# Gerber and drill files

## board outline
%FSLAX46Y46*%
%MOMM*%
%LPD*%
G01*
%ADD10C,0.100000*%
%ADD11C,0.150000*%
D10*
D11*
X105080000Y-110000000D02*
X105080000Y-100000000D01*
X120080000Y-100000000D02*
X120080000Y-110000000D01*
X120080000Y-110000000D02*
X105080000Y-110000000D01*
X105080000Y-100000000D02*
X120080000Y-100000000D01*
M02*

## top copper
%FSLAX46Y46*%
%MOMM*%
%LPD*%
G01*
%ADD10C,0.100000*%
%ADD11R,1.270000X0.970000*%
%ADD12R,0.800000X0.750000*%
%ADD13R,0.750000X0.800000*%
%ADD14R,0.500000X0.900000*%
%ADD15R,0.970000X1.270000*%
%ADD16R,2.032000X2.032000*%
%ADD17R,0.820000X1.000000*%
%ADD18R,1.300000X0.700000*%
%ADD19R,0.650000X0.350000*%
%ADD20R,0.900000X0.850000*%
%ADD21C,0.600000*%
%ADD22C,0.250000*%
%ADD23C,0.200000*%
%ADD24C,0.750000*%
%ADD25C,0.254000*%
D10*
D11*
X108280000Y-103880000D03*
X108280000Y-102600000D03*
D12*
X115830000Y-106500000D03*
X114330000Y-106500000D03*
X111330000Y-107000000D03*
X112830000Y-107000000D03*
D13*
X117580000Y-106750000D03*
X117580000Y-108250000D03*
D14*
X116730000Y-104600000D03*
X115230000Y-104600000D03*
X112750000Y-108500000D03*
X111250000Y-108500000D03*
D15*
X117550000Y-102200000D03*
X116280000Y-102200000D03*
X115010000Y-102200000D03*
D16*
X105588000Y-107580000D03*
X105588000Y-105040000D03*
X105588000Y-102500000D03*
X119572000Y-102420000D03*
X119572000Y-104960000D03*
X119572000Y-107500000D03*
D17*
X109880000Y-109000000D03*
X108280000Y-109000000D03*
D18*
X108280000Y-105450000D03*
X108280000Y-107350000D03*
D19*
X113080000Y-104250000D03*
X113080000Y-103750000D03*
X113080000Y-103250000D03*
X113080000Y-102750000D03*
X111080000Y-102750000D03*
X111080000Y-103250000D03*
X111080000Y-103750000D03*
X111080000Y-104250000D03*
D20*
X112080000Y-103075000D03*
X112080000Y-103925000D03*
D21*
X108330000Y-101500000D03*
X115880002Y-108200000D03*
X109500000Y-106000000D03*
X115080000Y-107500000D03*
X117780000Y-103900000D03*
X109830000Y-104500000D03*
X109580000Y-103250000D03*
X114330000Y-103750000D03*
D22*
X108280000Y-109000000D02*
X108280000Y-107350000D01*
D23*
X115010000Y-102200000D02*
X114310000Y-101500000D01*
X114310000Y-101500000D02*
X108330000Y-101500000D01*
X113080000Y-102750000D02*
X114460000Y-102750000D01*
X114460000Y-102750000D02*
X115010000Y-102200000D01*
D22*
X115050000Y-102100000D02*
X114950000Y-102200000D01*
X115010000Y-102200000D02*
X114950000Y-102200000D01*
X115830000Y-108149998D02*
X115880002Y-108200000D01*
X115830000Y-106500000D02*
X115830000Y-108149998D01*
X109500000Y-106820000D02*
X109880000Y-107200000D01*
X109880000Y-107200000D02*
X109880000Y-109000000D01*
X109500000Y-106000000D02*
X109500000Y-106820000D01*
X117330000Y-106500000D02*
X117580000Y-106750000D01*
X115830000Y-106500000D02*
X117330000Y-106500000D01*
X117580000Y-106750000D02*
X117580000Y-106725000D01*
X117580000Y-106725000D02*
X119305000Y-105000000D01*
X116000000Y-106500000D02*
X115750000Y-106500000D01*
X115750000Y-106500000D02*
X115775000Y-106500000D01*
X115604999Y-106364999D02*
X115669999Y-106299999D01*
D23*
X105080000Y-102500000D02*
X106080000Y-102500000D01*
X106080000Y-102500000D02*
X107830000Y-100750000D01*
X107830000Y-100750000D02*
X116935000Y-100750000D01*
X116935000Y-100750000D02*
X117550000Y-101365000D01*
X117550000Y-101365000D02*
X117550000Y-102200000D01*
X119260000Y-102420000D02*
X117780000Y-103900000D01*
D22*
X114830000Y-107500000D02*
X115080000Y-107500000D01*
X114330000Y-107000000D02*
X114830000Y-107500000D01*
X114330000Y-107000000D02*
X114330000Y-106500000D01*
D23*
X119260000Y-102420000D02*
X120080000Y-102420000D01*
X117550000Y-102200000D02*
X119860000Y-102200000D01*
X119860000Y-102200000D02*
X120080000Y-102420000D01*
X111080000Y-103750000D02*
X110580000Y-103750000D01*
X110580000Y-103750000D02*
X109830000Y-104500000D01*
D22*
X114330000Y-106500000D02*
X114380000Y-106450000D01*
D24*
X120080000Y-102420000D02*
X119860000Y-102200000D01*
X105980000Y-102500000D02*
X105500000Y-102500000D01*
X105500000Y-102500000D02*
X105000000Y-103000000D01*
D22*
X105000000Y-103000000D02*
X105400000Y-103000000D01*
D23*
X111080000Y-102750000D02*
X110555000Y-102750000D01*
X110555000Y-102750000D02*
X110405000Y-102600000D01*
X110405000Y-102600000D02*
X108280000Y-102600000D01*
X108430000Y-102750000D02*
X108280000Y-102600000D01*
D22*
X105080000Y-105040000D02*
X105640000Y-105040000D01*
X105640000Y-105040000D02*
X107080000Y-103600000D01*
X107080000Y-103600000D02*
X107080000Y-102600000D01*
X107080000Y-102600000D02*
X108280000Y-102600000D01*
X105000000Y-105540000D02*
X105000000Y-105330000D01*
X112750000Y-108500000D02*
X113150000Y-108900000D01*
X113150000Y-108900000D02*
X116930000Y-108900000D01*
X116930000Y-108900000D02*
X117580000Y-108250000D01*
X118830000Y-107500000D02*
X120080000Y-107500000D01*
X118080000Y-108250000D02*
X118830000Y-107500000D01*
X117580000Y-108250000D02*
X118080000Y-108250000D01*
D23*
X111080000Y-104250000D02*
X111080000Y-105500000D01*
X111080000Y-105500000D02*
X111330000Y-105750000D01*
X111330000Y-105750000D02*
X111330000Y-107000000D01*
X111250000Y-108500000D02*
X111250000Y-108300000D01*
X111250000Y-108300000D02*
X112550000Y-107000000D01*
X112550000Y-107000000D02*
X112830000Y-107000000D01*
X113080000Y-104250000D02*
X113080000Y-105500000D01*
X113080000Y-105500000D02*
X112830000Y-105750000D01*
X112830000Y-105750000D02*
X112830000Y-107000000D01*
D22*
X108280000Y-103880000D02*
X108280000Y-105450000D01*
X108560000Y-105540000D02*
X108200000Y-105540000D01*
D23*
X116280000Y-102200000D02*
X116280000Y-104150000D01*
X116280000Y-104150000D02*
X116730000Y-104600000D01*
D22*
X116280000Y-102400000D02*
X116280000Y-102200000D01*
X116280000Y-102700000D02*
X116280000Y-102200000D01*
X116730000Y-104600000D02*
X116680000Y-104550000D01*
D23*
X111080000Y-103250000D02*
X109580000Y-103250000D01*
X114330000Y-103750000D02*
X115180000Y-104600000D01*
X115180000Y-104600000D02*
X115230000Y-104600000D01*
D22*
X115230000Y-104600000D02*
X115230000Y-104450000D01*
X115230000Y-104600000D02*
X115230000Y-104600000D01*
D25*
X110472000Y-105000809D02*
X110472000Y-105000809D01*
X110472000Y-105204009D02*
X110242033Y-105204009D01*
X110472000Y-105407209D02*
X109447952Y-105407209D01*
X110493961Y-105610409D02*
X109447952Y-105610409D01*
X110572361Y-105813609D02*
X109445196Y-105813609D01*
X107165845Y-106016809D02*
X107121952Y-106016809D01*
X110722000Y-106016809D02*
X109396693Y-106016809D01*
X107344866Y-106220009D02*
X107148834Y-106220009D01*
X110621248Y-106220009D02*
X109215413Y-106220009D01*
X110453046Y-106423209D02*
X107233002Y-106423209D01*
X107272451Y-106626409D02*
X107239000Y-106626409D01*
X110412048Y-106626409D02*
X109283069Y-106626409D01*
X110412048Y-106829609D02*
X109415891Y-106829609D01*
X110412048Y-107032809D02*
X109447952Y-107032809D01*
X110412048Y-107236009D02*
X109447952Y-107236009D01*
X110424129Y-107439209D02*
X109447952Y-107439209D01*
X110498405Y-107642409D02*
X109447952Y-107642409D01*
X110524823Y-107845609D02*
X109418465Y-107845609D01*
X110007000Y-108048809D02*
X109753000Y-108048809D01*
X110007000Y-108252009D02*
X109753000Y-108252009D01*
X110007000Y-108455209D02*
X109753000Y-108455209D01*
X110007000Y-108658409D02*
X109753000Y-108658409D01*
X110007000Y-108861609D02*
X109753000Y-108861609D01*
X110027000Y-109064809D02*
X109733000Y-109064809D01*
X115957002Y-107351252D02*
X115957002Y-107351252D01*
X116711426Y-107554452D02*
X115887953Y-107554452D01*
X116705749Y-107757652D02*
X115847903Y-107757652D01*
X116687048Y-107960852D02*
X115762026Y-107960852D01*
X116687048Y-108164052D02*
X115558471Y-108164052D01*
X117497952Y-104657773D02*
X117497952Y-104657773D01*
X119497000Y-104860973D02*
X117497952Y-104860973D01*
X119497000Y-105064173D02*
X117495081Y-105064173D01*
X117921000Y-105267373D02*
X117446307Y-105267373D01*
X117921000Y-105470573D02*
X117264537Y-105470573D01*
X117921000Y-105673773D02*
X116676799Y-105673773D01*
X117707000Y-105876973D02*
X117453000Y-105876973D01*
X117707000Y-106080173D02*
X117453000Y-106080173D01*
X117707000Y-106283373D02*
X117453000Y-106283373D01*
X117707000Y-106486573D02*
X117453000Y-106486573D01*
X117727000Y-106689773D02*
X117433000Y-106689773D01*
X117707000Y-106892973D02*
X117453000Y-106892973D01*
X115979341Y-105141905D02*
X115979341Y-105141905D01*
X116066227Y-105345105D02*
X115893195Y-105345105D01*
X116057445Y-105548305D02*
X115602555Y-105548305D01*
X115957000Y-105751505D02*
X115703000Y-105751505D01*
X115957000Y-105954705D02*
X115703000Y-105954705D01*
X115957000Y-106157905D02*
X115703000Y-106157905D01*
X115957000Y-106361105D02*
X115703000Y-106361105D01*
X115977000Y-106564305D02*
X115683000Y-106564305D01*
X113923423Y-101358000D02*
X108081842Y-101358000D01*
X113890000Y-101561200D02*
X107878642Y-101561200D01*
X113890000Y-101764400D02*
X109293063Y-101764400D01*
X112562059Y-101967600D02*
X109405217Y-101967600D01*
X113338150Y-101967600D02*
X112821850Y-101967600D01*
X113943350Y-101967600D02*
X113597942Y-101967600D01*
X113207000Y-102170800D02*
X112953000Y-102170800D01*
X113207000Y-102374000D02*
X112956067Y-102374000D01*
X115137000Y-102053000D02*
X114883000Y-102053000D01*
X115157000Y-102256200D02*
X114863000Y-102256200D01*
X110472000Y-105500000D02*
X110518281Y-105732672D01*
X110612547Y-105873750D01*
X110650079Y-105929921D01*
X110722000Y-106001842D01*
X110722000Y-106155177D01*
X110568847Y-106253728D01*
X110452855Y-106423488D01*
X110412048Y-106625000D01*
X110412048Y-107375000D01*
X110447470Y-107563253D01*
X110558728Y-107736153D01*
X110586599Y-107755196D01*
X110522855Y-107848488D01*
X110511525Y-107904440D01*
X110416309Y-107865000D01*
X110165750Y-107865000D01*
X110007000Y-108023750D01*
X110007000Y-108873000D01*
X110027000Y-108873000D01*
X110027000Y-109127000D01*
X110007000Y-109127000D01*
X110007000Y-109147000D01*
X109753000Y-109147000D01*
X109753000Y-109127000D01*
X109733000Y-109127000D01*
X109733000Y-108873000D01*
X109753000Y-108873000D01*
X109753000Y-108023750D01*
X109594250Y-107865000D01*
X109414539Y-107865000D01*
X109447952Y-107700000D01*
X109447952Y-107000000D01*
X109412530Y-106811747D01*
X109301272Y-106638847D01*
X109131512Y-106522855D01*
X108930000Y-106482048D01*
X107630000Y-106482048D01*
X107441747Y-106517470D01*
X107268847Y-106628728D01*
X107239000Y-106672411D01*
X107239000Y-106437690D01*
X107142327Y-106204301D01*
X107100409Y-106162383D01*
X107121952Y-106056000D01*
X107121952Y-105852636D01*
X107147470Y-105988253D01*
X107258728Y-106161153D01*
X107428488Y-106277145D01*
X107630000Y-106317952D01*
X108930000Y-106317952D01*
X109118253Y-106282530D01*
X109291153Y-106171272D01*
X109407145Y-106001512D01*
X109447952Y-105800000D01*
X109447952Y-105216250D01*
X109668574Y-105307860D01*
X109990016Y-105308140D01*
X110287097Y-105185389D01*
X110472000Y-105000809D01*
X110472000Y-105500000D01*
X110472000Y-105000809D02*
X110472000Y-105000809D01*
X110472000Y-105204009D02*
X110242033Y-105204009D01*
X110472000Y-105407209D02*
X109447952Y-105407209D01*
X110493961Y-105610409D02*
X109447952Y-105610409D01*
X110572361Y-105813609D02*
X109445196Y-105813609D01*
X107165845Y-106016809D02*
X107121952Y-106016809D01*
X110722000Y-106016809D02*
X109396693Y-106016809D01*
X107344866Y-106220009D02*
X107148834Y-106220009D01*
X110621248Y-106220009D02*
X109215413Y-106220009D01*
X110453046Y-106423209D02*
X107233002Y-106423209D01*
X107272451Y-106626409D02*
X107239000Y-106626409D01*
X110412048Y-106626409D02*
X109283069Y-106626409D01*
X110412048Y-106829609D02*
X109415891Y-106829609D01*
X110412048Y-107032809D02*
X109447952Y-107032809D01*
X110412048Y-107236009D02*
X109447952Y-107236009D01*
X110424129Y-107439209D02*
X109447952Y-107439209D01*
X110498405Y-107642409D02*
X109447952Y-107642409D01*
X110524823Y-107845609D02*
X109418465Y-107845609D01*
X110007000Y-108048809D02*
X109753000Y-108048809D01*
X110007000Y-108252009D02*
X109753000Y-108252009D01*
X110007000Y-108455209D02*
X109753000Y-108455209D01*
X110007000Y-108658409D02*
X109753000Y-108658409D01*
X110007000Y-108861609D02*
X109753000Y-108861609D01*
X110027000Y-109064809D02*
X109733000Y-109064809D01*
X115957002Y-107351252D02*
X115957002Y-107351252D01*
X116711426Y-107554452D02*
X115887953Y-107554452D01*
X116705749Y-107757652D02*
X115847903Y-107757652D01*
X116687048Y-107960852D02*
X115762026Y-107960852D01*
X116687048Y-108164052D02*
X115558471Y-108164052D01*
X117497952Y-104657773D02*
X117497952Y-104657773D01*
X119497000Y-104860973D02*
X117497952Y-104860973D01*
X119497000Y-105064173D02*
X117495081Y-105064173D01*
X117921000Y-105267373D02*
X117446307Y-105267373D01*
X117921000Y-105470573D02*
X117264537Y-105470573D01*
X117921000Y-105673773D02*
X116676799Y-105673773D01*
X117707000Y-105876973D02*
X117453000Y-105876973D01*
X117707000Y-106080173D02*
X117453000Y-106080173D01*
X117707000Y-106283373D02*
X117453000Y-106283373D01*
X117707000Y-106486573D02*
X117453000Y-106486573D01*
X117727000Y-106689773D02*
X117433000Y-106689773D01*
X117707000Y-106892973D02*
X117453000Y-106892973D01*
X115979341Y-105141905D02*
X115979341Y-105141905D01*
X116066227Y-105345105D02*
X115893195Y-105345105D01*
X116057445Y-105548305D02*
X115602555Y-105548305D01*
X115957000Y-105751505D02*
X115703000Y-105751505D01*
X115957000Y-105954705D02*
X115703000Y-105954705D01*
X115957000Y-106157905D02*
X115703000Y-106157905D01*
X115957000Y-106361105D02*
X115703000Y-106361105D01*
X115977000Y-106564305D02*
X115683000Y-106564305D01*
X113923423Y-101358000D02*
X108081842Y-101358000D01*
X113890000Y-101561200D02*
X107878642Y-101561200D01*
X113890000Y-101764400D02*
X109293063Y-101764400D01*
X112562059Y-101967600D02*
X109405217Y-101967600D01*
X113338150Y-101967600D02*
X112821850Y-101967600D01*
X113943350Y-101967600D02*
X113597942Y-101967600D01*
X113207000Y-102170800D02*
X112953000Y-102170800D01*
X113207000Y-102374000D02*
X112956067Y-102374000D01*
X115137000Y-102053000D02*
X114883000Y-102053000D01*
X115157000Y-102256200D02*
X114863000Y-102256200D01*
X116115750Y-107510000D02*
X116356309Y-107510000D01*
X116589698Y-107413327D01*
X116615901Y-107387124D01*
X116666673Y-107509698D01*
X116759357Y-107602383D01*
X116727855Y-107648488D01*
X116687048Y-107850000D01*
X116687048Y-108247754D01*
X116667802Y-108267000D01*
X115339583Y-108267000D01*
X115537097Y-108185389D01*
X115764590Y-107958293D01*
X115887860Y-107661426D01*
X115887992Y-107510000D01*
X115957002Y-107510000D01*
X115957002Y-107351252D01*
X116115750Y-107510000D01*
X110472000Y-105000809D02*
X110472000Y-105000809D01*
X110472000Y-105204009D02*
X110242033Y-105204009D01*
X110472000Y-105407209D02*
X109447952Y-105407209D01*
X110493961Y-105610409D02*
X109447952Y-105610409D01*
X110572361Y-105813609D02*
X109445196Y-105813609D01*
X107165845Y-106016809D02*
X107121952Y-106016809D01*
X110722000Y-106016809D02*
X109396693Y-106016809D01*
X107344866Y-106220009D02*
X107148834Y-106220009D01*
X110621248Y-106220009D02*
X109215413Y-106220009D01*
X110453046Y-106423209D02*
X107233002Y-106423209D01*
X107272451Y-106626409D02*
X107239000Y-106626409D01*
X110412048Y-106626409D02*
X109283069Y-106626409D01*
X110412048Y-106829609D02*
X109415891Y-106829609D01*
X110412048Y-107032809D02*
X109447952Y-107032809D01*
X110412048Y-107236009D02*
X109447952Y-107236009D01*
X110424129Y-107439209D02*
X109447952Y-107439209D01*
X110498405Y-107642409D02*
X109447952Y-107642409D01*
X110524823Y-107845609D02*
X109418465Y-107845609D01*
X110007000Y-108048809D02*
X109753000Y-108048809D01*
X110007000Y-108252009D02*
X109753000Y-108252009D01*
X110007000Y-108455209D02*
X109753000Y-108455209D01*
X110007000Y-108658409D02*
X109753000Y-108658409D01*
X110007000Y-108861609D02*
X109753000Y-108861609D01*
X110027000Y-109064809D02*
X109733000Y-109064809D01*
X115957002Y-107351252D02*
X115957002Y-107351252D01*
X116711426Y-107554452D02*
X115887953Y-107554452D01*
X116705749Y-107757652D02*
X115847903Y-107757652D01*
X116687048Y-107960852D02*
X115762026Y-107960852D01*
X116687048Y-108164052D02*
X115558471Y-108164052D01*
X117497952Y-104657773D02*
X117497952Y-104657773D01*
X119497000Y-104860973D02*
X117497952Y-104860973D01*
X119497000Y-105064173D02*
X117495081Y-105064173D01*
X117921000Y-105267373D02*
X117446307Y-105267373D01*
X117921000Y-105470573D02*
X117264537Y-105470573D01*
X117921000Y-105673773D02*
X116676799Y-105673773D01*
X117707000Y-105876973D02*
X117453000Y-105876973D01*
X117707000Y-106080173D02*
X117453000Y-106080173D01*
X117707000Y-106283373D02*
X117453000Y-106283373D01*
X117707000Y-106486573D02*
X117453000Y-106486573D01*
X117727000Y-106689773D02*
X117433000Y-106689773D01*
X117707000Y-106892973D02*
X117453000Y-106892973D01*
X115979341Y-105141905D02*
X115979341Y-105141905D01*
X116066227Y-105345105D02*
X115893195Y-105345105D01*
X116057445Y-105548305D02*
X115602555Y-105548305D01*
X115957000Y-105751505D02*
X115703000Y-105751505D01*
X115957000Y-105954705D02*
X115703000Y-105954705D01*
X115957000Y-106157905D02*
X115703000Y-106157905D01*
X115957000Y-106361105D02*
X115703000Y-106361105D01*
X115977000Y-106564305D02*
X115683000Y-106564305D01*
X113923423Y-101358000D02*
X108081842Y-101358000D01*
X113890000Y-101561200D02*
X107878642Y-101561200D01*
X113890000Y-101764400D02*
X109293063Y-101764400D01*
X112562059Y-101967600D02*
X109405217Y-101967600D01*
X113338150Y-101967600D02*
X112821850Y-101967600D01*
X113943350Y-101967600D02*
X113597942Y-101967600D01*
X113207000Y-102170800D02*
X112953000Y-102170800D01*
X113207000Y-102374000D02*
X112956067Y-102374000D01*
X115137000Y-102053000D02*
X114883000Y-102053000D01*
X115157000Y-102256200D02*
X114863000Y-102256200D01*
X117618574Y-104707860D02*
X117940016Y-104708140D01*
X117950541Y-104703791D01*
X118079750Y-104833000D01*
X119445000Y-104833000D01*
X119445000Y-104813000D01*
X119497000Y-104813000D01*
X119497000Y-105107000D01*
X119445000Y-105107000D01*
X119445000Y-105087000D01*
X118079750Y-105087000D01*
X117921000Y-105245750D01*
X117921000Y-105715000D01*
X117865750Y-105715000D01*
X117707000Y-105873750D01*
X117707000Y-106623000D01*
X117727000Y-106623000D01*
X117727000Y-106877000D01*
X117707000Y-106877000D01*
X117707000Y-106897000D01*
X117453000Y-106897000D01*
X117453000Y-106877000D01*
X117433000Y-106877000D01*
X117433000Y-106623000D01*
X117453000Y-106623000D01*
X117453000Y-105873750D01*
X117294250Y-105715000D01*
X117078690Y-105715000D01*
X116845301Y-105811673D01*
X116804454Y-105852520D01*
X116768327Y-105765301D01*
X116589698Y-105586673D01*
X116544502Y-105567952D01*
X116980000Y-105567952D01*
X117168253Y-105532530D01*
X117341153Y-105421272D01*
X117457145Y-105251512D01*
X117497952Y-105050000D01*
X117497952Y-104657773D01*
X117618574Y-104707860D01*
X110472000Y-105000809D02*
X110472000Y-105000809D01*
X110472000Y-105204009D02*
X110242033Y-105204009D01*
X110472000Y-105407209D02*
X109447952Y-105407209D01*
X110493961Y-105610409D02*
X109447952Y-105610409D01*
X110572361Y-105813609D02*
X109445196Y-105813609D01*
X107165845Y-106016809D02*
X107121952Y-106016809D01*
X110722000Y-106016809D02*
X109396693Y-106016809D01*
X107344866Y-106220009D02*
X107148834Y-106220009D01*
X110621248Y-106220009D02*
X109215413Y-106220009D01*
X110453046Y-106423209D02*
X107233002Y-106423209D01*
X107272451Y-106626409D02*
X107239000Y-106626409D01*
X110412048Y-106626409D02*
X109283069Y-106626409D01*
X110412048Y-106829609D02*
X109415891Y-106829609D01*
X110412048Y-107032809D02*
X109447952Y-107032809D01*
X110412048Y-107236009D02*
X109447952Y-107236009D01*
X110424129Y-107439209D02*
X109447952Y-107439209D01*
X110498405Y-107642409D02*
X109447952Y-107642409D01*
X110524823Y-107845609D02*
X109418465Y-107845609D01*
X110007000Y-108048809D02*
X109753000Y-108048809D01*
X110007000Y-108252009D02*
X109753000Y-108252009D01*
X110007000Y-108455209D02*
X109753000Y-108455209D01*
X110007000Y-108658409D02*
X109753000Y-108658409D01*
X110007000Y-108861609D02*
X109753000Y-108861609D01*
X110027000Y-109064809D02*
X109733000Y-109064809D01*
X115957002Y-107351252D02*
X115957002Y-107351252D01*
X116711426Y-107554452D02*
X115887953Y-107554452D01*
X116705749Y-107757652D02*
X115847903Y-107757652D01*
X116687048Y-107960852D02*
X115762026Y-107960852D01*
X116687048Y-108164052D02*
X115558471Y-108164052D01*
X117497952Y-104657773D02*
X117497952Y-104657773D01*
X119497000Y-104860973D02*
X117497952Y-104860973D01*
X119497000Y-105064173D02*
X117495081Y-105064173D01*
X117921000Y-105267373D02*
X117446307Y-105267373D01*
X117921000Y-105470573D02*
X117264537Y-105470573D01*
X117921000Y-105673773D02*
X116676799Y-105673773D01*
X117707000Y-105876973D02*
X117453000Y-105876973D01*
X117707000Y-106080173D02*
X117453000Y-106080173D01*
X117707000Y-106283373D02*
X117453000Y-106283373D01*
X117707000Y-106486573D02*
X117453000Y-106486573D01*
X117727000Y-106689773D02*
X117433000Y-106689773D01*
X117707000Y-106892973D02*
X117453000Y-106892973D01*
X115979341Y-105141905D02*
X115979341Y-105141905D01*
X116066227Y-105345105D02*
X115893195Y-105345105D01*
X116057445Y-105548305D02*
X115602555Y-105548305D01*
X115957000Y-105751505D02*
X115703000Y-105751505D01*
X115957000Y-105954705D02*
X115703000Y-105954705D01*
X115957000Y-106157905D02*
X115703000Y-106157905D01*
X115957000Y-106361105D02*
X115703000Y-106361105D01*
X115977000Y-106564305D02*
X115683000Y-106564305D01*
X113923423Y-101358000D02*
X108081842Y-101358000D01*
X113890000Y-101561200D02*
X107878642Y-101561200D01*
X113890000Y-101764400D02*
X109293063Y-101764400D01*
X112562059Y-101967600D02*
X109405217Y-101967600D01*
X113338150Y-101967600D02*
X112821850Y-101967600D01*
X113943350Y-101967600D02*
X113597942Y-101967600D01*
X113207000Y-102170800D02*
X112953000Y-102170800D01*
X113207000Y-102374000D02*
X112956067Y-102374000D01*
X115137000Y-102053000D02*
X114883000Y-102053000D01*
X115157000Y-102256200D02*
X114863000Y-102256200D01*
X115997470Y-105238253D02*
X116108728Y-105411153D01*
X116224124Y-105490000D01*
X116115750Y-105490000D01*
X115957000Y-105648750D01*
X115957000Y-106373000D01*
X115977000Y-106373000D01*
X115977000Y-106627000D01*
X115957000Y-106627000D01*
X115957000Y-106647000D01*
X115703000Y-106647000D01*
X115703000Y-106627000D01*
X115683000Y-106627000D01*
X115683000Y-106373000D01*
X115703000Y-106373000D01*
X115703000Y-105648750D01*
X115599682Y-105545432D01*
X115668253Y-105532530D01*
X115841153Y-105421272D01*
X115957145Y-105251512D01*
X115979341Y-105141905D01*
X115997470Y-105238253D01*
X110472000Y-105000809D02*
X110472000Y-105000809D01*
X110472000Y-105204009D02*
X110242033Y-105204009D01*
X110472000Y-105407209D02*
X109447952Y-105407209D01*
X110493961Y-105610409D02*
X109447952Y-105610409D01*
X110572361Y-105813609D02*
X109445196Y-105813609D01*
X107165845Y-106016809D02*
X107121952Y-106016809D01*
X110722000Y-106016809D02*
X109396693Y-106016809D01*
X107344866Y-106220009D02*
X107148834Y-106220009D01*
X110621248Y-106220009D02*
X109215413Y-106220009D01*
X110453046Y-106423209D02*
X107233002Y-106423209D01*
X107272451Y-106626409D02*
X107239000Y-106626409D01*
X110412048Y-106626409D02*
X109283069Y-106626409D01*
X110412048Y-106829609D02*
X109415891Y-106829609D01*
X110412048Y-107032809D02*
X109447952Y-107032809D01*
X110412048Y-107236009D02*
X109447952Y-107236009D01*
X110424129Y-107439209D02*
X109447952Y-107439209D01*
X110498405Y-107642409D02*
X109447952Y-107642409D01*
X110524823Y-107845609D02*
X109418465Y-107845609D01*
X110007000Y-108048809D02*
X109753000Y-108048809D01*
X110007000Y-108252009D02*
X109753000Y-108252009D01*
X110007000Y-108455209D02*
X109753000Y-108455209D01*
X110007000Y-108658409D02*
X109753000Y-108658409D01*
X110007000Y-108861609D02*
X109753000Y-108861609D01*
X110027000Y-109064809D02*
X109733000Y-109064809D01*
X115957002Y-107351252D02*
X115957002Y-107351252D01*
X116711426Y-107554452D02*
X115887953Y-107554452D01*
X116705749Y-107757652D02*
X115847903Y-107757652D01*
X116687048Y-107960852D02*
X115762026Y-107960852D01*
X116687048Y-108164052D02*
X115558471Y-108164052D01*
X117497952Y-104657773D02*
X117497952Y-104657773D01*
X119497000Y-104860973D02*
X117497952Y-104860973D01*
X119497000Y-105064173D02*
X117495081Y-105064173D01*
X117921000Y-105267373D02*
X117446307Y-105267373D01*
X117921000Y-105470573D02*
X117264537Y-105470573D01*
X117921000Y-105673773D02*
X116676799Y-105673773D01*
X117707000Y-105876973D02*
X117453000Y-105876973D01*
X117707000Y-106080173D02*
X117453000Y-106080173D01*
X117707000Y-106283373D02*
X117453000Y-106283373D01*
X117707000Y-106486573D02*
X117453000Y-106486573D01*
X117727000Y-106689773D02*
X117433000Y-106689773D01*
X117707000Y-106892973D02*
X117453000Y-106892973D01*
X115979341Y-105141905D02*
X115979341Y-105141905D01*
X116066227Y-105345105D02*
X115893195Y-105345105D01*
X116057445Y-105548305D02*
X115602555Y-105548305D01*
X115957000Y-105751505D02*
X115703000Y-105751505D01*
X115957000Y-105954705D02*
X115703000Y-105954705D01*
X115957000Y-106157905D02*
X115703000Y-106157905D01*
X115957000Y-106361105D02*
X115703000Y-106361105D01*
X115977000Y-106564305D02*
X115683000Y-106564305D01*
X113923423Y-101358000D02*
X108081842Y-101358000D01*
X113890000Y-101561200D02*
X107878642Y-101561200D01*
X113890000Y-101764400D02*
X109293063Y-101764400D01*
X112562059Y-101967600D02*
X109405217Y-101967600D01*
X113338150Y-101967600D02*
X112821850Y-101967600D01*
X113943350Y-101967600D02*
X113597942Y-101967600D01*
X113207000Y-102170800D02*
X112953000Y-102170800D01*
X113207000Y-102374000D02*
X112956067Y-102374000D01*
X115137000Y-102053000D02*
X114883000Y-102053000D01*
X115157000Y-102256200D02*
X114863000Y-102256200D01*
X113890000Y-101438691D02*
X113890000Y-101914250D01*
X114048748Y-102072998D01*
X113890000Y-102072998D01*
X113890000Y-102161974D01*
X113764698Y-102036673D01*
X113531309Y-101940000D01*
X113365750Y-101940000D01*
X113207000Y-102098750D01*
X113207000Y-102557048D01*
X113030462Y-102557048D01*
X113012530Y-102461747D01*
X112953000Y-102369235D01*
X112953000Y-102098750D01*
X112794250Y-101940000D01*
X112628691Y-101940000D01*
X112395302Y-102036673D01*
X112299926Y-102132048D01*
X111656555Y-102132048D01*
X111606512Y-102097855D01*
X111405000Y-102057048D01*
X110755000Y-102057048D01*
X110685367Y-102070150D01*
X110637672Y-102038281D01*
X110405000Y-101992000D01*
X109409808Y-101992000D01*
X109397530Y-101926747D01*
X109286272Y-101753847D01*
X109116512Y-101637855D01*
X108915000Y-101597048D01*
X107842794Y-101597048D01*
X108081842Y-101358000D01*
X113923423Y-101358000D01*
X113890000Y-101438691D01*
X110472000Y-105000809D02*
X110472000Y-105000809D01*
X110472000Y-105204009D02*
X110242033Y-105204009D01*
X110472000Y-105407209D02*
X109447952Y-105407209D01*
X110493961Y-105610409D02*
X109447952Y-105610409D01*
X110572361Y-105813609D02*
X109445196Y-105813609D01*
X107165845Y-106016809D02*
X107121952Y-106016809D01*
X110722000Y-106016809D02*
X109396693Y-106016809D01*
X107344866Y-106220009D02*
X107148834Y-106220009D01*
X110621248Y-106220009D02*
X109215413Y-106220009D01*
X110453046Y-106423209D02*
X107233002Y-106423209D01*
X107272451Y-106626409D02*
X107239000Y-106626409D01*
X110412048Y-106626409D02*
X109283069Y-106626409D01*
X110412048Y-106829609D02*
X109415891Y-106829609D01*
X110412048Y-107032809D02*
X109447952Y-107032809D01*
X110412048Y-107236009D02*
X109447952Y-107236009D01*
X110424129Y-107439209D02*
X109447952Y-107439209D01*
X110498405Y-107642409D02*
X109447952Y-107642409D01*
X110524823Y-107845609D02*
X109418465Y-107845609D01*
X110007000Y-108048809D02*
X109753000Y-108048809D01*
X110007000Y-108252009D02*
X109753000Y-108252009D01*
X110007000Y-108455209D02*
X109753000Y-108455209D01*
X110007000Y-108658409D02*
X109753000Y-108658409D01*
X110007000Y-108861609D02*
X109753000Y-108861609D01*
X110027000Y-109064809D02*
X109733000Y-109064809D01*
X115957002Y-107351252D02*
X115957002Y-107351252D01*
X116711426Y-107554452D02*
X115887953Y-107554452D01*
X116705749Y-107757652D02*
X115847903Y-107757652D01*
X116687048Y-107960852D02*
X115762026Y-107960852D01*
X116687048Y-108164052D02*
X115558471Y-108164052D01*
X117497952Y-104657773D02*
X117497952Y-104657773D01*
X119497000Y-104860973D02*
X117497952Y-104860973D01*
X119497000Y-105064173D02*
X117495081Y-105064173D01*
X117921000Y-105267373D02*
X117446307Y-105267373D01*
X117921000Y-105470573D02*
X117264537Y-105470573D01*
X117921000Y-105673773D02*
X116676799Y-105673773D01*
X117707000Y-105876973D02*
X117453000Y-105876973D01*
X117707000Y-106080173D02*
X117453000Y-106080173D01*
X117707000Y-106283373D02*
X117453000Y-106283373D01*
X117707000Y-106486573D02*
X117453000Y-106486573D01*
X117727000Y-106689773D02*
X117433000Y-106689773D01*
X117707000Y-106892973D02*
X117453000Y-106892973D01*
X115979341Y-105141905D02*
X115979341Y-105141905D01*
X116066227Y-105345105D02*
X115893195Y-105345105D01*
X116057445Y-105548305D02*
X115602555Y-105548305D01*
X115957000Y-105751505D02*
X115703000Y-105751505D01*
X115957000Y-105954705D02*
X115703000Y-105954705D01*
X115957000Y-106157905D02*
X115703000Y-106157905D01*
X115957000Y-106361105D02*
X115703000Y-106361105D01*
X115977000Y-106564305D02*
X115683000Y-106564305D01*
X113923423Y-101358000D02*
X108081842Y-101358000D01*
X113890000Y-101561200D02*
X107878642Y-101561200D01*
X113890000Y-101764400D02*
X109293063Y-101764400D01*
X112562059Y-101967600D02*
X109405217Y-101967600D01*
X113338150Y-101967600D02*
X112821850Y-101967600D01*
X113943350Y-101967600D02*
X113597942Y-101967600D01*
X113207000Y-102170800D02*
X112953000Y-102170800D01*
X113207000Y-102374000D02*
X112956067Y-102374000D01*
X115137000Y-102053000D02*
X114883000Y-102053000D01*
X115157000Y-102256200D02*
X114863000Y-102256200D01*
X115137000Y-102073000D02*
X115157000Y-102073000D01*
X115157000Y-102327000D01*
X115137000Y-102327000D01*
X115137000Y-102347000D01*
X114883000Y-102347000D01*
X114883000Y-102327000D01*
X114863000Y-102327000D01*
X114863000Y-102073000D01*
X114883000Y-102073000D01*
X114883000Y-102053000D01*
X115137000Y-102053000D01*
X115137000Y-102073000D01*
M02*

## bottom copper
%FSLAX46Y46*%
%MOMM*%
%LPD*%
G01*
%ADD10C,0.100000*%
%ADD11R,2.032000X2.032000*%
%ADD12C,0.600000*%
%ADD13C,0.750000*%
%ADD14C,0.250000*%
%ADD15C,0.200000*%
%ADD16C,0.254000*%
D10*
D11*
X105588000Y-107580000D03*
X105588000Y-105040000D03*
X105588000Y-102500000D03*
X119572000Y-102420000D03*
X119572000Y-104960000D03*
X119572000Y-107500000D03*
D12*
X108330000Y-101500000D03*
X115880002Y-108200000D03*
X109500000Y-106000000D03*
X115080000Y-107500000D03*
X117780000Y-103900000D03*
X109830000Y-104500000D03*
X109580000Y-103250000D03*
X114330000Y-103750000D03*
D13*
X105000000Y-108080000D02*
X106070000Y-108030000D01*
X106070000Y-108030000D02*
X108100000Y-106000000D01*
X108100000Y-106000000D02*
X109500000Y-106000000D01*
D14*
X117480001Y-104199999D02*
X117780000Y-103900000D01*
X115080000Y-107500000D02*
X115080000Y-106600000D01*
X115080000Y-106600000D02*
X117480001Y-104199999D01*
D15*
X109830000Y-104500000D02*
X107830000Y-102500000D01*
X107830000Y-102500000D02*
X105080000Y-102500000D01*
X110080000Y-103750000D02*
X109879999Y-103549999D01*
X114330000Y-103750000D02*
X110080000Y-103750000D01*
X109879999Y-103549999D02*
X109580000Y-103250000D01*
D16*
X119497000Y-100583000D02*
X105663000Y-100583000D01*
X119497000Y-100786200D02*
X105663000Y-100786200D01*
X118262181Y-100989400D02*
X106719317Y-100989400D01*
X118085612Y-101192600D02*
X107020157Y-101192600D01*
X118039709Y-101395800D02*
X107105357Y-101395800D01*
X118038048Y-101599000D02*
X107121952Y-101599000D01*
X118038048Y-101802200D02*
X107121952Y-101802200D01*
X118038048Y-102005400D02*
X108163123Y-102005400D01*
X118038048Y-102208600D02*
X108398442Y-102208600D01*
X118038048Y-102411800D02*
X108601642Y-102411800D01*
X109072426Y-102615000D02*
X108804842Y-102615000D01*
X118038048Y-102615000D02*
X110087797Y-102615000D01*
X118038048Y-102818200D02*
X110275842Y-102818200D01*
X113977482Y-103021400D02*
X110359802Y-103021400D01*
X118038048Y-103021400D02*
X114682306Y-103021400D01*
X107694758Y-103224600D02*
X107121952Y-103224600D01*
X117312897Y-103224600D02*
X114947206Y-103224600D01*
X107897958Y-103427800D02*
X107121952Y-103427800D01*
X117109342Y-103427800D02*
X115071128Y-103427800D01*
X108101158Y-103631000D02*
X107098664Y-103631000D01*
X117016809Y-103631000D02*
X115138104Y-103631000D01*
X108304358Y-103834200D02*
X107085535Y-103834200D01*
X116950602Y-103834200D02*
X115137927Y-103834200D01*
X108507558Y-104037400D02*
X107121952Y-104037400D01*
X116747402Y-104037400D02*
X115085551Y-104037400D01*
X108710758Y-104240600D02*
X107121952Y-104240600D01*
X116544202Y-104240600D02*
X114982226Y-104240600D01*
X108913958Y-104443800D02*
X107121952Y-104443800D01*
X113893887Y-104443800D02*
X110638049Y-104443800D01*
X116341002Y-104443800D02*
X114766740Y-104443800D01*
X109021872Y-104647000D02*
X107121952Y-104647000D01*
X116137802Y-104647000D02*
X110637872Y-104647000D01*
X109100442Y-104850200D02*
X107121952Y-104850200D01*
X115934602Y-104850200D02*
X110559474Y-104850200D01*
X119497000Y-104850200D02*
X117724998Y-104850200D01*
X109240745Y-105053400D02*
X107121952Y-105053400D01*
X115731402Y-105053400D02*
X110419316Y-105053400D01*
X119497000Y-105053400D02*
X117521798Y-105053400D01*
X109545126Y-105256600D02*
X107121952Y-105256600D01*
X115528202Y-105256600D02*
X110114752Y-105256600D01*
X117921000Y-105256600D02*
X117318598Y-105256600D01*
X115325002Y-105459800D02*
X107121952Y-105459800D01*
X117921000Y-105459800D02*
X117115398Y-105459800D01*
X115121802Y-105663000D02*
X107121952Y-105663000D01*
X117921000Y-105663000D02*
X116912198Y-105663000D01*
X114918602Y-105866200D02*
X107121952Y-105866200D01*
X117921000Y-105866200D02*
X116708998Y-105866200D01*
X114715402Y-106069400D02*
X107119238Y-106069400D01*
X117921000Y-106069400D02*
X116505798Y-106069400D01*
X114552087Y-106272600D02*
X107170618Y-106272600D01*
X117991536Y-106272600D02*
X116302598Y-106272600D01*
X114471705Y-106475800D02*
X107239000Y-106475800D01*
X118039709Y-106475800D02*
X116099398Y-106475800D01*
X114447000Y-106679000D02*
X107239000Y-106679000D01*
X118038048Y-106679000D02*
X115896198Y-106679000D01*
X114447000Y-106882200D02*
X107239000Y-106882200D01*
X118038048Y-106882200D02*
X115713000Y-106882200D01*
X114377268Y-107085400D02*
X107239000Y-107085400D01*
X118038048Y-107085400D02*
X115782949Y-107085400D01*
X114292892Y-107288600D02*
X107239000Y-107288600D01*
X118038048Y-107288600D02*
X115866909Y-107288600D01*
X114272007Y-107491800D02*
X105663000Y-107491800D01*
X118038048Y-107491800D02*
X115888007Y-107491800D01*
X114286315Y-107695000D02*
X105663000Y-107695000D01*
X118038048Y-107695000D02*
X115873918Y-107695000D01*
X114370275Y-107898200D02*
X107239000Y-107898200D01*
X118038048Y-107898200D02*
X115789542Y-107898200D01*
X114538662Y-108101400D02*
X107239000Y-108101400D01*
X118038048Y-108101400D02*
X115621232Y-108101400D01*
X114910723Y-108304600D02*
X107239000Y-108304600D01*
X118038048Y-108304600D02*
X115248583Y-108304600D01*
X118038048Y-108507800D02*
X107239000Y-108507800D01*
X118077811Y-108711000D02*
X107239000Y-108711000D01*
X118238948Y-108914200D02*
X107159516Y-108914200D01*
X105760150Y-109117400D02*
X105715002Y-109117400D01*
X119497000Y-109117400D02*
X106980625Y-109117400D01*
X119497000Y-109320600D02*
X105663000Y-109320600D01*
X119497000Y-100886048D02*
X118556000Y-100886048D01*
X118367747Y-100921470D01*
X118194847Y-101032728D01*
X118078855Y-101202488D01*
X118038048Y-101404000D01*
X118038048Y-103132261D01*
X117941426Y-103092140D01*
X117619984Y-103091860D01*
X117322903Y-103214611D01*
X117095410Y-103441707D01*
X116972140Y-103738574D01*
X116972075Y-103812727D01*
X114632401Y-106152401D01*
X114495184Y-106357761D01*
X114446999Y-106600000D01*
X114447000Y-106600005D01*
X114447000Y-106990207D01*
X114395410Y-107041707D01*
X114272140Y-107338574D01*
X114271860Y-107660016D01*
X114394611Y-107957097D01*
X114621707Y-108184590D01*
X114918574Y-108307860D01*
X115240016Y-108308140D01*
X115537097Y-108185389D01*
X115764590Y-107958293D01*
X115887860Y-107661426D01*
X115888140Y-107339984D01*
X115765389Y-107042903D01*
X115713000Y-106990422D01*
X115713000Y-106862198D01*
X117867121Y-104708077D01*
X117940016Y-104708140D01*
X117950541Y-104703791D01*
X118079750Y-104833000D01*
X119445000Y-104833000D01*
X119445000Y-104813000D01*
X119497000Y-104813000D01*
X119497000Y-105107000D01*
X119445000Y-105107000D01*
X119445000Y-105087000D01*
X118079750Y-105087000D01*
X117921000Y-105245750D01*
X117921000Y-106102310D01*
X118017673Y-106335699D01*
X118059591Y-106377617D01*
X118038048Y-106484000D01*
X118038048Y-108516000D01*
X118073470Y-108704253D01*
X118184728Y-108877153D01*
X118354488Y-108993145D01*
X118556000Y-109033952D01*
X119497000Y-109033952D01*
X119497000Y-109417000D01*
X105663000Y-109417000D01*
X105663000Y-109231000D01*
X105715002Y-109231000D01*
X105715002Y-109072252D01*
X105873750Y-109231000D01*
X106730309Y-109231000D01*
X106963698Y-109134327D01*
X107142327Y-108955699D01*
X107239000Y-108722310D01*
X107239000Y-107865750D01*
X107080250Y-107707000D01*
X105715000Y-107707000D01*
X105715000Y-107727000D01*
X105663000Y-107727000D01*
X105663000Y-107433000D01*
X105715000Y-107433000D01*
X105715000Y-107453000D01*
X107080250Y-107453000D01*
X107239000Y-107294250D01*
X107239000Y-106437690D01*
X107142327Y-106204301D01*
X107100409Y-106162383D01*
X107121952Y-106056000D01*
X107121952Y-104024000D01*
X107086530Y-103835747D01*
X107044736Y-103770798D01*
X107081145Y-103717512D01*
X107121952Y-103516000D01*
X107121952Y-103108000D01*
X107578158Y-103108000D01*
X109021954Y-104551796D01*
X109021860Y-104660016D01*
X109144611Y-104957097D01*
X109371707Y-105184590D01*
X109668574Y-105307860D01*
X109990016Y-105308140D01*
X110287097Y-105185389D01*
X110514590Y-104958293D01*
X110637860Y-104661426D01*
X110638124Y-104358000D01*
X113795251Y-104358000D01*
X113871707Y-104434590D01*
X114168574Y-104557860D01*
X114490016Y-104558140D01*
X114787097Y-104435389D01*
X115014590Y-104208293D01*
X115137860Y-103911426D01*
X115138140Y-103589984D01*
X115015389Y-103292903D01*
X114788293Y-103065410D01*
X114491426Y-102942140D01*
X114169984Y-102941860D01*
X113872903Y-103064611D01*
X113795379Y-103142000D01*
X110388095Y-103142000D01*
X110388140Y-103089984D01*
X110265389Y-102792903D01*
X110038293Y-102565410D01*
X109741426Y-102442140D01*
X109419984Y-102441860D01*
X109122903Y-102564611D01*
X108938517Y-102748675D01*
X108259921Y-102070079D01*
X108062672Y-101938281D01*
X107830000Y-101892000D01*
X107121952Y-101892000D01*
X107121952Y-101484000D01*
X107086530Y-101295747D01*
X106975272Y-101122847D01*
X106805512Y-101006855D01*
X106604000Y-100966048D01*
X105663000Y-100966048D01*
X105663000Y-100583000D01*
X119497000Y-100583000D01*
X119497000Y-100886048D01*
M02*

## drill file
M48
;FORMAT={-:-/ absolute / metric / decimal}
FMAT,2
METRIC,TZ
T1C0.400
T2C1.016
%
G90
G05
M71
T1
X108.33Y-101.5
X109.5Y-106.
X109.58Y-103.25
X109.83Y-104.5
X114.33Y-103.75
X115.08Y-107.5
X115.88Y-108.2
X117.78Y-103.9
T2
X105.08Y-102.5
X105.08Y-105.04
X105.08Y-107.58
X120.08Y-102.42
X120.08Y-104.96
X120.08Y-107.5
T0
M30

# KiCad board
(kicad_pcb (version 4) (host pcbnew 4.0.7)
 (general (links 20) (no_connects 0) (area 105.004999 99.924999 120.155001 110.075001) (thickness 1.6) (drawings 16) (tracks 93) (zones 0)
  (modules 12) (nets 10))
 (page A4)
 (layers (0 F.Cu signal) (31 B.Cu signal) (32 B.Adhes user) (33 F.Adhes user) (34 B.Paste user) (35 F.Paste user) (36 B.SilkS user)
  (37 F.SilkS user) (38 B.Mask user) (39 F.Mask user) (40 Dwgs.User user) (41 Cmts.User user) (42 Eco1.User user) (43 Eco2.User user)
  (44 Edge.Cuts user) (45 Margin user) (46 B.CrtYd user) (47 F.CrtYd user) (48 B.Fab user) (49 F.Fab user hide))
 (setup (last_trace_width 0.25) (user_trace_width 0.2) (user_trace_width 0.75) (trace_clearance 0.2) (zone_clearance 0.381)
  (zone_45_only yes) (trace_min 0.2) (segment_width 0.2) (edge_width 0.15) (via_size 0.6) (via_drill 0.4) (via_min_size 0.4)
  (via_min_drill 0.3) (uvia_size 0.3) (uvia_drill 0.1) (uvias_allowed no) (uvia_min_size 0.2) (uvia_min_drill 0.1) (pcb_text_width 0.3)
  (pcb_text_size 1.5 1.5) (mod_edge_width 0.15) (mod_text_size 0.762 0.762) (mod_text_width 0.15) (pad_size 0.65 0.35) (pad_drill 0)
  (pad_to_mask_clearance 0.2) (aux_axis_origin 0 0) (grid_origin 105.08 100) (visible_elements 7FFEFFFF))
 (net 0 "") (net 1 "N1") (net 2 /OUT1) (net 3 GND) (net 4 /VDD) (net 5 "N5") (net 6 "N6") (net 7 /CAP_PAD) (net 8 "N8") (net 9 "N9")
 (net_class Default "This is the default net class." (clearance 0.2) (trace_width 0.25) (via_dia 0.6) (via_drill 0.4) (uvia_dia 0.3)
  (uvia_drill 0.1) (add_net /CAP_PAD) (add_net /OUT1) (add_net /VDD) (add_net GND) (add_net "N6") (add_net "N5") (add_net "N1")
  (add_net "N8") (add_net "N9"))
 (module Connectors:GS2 (layer F.Cu) (at 108.28 103.24 180)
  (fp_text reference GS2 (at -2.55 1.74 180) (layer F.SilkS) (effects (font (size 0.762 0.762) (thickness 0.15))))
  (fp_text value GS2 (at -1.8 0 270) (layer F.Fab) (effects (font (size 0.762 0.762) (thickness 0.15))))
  (pad 1 smd rect (at 0 -0.64 180) (size 1.27 0.97) (layers F.Cu F.Paste F.Mask) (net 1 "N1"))
  (pad 2 smd rect (at 0 0.64 180) (size 1.27 0.97) (layers F.Cu F.Paste F.Mask) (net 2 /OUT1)))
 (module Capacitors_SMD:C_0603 (layer F.Cu) (at 115.08 106.5)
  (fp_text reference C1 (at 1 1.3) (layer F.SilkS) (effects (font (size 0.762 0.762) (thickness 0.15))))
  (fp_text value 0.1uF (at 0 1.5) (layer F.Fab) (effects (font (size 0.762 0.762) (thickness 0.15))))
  (pad 2 smd rect (at 0.75 0) (size 0.8 0.75) (layers F.Cu F.Paste F.Mask) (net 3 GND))
  (pad 1 smd rect (at -0.75 0) (size 0.8 0.75) (layers F.Cu F.Paste F.Mask) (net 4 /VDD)))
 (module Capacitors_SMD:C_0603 (layer F.Cu) (at 112.08 107 180)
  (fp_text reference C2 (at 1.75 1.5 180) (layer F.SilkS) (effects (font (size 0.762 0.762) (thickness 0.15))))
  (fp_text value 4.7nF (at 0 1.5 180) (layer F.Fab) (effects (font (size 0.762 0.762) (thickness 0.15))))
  (pad 2 smd rect (at 0.75 0 180) (size 0.8 0.75) (layers F.Cu F.Paste F.Mask) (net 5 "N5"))
  (pad 1 smd rect (at -0.75 0 180) (size 0.8 0.75) (layers F.Cu F.Paste F.Mask) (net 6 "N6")))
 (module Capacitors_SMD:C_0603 (layer F.Cu) (at 117.58 107.5 90)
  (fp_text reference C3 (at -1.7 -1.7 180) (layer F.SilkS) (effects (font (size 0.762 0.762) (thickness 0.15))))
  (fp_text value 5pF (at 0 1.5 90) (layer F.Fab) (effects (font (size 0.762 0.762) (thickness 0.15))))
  (pad 2 smd rect (at 0.75 0 90) (size 0.8 0.75) (layers F.Cu F.Paste F.Mask) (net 3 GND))
  (pad 1 smd rect (at -0.75 0 90) (size 0.8 0.75) (layers F.Cu F.Paste F.Mask) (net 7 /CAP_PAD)))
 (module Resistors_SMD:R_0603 (layer F.Cu) (at 115.98 104.6 180)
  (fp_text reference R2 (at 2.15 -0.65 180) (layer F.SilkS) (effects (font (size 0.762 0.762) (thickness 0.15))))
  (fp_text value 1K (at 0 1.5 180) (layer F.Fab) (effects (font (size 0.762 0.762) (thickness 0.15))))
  (pad 1 smd rect (at -0.75 0 180) (size 0.5 0.9) (layers F.Cu F.Paste F.Mask) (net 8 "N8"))
  (pad 2 smd rect (at 0.75 0 180) (size 0.5 0.9) (layers F.Cu F.Paste F.Mask) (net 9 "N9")))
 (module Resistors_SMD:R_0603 (layer F.Cu) (at 112 108.5 180)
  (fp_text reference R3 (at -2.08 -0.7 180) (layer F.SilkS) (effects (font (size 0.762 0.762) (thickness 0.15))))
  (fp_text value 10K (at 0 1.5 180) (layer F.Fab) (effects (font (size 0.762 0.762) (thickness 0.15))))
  (pad 1 smd rect (at -0.75 0 180) (size 0.5 0.9) (layers F.Cu F.Paste F.Mask) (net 7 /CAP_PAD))
  (pad 2 smd rect (at 0.75 0 180) (size 0.5 0.9) (layers F.Cu F.Paste F.Mask) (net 6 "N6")))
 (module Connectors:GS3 (layer F.Cu) (at 116.28 102.2 270)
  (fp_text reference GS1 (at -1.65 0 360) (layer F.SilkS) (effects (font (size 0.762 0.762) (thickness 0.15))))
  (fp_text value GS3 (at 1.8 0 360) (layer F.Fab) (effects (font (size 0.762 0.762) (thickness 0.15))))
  (pad 1 smd rect (at 0 -1.27 270) (size 1.27 0.97) (layers F.Cu F.Paste F.Mask) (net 4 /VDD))
  (pad 2 smd rect (at 0 0 270) (size 1.27 0.97) (layers F.Cu F.Paste F.Mask) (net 8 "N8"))
  (pad 3 smd rect (at 0 1.27 270) (size 1.27 0.97) (layers F.Cu F.Paste F.Mask) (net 3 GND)))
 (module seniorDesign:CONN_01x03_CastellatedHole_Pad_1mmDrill (layer F.Cu) (at 105.08 102.5)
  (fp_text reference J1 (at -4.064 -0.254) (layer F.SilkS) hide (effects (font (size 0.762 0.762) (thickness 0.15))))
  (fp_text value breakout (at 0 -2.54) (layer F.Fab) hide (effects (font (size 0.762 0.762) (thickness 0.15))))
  (pad 3 thru_hole rect (at 0 5.08) (size 2.032 2.032) (drill 1.016 (offset 0.508 0)) (layers *.Cu *.Mask B.Paste) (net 3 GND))
  (pad 2 thru_hole rect (at 0 2.54) (size 2.032 2.032) (drill 1.016 (offset 0.508 0)) (layers *.Cu *.Mask B.Paste) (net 2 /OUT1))
  (pad 1 thru_hole rect (at 0 0) (size 2.032 2.032) (drill 1.016 (offset 0.508 0)) (layers *.Cu *.Mask B.Paste) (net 4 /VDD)))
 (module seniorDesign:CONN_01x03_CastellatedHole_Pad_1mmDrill (layer F.Cu) (at 120.08 107.5 180)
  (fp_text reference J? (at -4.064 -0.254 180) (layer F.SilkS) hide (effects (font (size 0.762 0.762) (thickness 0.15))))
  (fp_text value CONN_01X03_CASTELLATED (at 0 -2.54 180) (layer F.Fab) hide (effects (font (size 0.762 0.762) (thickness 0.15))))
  (pad 4 thru_hole rect (at 0 5.08 180) (size 2.032 2.032) (drill 1.016 (offset 0.508 0)) (layers *.Cu *.Mask B.Paste) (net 4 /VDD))
  (pad 5 thru_hole rect (at 0 2.54 180) (size 2.032 2.032) (drill 1.016 (offset 0.508 0)) (layers *.Cu *.Mask B.Paste) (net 3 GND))
  (pad 6 thru_hole rect (at 0 0 180) (size 2.032 2.032) (drill 1.016 (offset 0.508 0)) (layers *.Cu *.Mask B.Paste) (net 7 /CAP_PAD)))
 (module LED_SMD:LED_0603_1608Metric (layer F.Cu) (at 109.08 109 180)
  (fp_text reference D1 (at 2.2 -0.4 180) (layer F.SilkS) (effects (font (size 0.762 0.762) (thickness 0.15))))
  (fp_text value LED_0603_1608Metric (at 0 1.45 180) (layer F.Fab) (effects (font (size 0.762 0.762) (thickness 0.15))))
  (pad 1 smd rect (at -0.8 0 180) (size 0.82 1) (layers F.Cu F.Paste F.Mask) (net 3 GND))
  (pad 2 smd rect (at 0.8 0 180) (size 0.82 1) (layers F.Cu F.Paste F.Mask)))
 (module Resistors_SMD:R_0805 (layer F.Cu) (at 108.28 106.4 270)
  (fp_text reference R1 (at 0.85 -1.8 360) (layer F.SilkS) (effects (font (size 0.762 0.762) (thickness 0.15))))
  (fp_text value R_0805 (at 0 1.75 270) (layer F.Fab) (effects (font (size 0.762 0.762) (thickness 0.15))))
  (pad 1 smd rect (at -0.95 0 270) (size 0.7 1.3) (layers F.Cu F.Paste F.Mask) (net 1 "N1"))
  (pad 2 smd rect (at 0.95 0 270) (size 0.7 1.3) (layers F.Cu F.Paste F.Mask)))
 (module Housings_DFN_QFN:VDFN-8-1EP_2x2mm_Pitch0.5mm (layer F.Cu) (at 112.08 103.5 180)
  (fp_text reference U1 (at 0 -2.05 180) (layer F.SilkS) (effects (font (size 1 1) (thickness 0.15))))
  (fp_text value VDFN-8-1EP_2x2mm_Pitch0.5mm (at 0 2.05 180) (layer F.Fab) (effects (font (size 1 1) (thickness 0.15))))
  (pad 1 smd rect (at -1 -0.75 180) (size 0.65 0.35) (layers F.Cu F.Paste F.Mask) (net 6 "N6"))
  (pad 2 smd rect (at -1 -0.25 180) (size 0.65 0.35) (layers F.Cu F.Paste F.Mask))
  (pad 3 smd rect (at -1 0.25 180) (size 0.65 0.35) (layers F.Cu F.Paste F.Mask))
  (pad 4 smd rect (at -1 0.75 180) (size 0.65 0.35) (layers F.Cu F.Paste F.Mask) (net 3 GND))
  (pad 5 smd rect (at 1 0.75 180) (size 0.65 0.35) (layers F.Cu F.Paste F.Mask) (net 2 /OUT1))
  (pad 6 smd rect (at 1 0.25 180) (size 0.65 0.35) (layers F.Cu F.Paste F.Mask) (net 9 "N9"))
  (pad 7 smd rect (at 1 -0.25 180) (size 0.65 0.35) (layers F.Cu F.Paste F.Mask) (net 4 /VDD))
  (pad 8 smd rect (at 1 -0.75 180) (size 0.65 0.35) (layers F.Cu F.Paste F.Mask) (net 5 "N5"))
  (pad 9 smd rect (at 0 0.425 180) (size 0.9 0.85) (layers F.Cu F.Paste F.Mask) (solder_paste_margin_ratio -0.2))
  (pad 9 smd rect (at 0 -0.425 180) (size 0.9 0.85) (layers F.Cu F.Paste F.Mask) (solder_paste_margin_ratio -0.2)))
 (gr_line (start 105.08 110) (end 105.08 100) (angle 90) (layer Edge.Cuts) (width 0.15))
 (gr_line (start 120.08 100) (end 120.08 110) (angle 90) (layer Edge.Cuts) (width 0.15))
 (gr_line (start 120.08 110) (end 105.08 110) (angle 90) (layer Edge.Cuts) (width 0.15))
 (gr_line (start 105.08 100) (end 120.08 100) (angle 90) (layer Edge.Cuts) (width 0.15))
 (segment (start 108.28 109) (end 108.28 107.35) (width 0.25) (layer F.Cu) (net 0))
 (via (at 108.33 101.5) (size 0.6) (drill 0.4) (layers F.Cu B.Cu) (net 3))
 (segment (start 115.01 102.2) (end 114.31 101.5) (width 0.2) (layer F.Cu) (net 3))
 (segment (start 114.31 101.5) (end 108.33 101.5) (width 0.2) (layer F.Cu) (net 3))
 (segment (start 113.08 102.75) (end 114.46 102.75) (width 0.2) (layer F.Cu) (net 3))
 (segment (start 114.46 102.75) (end 115.01 102.2) (width 0.2) (layer F.Cu) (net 3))
 (segment (start 115.05 102.1) (end 114.95 102.2) (width 0.25) (layer F.Cu) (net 3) (status 30))
 (segment (start 115.01 102.2) (end 114.95 102.2) (width 0.25) (layer F.Cu) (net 3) (status 30))
 (segment (start 115.83 108.149998) (end 115.880002 108.2) (width 0.25) (layer F.Cu) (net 3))
 (segment (start 115.83 106.5) (end 115.83 108.149998) (width 0.25) (layer F.Cu) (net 3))
 (via (at 115.880002 108.2) (size 0.6) (drill 0.4) (layers F.Cu B.Cu) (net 3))
 (segment (start 109.5 106.82) (end 109.88 107.2) (width 0.25) (layer F.Cu) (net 3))
 (segment (start 109.88 107.2) (end 109.88 109) (width 0.25) (layer F.Cu) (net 3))
 (segment (start 109.5 106) (end 109.5 106.82) (width 0.25) (layer F.Cu) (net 3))
 (segment (start 117.33 106.5) (end 117.58 106.75) (width 0.25) (layer F.Cu) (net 3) (status 30))
 (segment (start 115.83 106.5) (end 117.33 106.5) (width 0.25) (layer F.Cu) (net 3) (status 20))
 (segment (start 117.58 106.75) (end 117.58 106.725) (width 0.25) (layer F.Cu) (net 3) (status 30))
 (segment (start 117.58 106.725) (end 119.305 105) (width 0.25) (layer F.Cu) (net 3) (status 10))
 (segment (start 116 106.5) (end 115.75 106.5) (width 0.25) (layer F.Cu) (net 3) (status 30))
 (segment (start 115.75 106.5) (end 115.775 106.5) (width 0.25) (layer F.Cu) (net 3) (status 30))
 (segment (start 105 108.08) (end 106.07 108.03) (width 0.75) (layer B.Cu) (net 3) (status 10))
 (segment (start 106.07 108.03) (end 108.1 106) (width 0.75) (layer B.Cu) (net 3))
 (segment (start 108.1 106) (end 109.5 106) (width 0.75) (layer B.Cu) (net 3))
 (via (at 109.5 106) (size 0.6) (drill 0.4) (layers F.Cu B.Cu) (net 3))
 (segment (start 115.604999 106.364999) (end 115.669999 106.299999) (width 0.25) (layer F.Cu) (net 3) (status 30))
 (segment (start 105.08 102.5) (end 106.08 102.5) (width 0.2) (layer F.Cu) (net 4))
 (segment (start 106.08 102.5) (end 107.83 100.75) (width 0.2) (layer F.Cu) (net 4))
 (segment (start 107.83 100.75) (end 116.935 100.75) (width 0.2) (layer F.Cu) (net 4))
 (segment (start 116.935 100.75) (end 117.55 101.365) (width 0.2) (layer F.Cu) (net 4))
 (segment (start 117.55 101.365) (end 117.55 102.2) (width 0.2) (layer F.Cu) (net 4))
 (segment (start 119.26 102.42) (end 117.78 103.9) (width 0.2) (layer F.Cu) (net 4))
 (via (at 115.08 107.5) (size 0.6) (drill 0.4) (layers F.Cu B.Cu) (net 4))
 (segment (start 114.83 107.5) (end 115.08 107.5) (width 0.25) (layer F.Cu) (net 4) (status 10))
 (segment (start 114.33 107) (end 114.83 107.5) (width 0.25) (layer F.Cu) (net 4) (status 20))
 (segment (start 114.33 107) (end 114.33 106.5) (width 0.25) (layer F.Cu) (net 4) (status 10))
 (via (at 117.78 103.9) (size 0.6) (drill 0.4) (layers F.Cu B.Cu) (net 4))
 (segment (start 117.480001 104.199999) (end 117.78 103.9) (width 0.25) (layer B.Cu) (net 4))
 (segment (start 115.08 107.5) (end 115.08 106.6) (width 0.25) (layer B.Cu) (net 4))
 (segment (start 115.08 106.6) (end 117.480001 104.199999) (width 0.25) (layer B.Cu) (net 4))
 (segment (start 119.26 102.42) (end 120.08 102.42) (width 0.2) (layer F.Cu) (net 4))
 (segment (start 117.55 102.2) (end 119.86 102.2) (width 0.2) (layer F.Cu) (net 4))
 (segment (start 119.86 102.2) (end 120.08 102.42) (width 0.2) (layer F.Cu) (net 4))
 (segment (start 109.83 104.5) (end 107.83 102.5) (width 0.2) (layer B.Cu) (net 4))
 (segment (start 107.83 102.5) (end 105.08 102.5) (width 0.2) (layer B.Cu) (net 4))
 (segment (start 111.08 103.75) (end 110.58 103.75) (width 0.2) (layer F.Cu) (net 4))
 (segment (start 110.58 103.75) (end 109.83 104.5) (width 0.2) (layer F.Cu) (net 4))
 (via (at 109.83 104.5) (size 0.6) (drill 0.4) (layers F.Cu B.Cu) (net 4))
 (segment (start 114.33 106.5) (end 114.38 106.45) (width 0.25) (layer F.Cu) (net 4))
 (segment (start 120.08 102.42) (end 119.86 102.2) (width 0.75) (layer F.Cu) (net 4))
 (segment (start 105.98 102.5) (end 105.5 102.5) (width 0.75) (layer F.Cu) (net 4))
 (segment (start 105.5 102.5) (end 105 103) (width 0.75) (layer F.Cu) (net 4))
 (segment (start 105 103) (end 105.4 103) (width 0.25) (layer F.Cu) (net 4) (status 30))
 (segment (start 111.08 102.75) (end 110.555 102.75) (width 0.2) (layer F.Cu) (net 2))
 (segment (start 110.555 102.75) (end 110.405 102.6) (width 0.2) (layer F.Cu) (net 2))
 (segment (start 110.405 102.6) (end 108.28 102.6) (width 0.2) (layer F.Cu) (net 2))
 (segment (start 108.43 102.75) (end 108.28 102.6) (width 0.2) (layer F.Cu) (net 2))
 (segment (start 105.08 105.04) (end 105.64 105.04) (width 0.25) (layer F.Cu) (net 2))
 (segment (start 105.64 105.04) (end 107.08 103.6) (width 0.25) (layer F.Cu) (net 2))
 (segment (start 107.08 103.6) (end 107.08 102.6) (width 0.25) (layer F.Cu) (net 2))
 (segment (start 107.08 102.6) (end 108.28 102.6) (width 0.25) (layer F.Cu) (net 2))
 (segment (start 105 105.54) (end 105 105.33) (width 0.25) (layer F.Cu) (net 2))
 (segment (start 112.75 108.5) (end 113.15 108.9) (width 0.25) (layer F.Cu) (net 7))
 (segment (start 113.15 108.9) (end 116.93 108.9) (width 0.25) (layer F.Cu) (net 7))
 (segment (start 116.93 108.9) (end 117.58 108.25) (width 0.25) (layer F.Cu) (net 7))
 (segment (start 118.83 107.5) (end 120.08 107.5) (width 0.25) (layer F.Cu) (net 7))
 (segment (start 118.08 108.25) (end 118.83 107.5) (width 0.25) (layer F.Cu) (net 7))
 (segment (start 117.58 108.25) (end 118.08 108.25) (width 0.25) (layer F.Cu) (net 7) (status 10))
 (segment (start 111.08 104.25) (end 111.08 105.5) (width 0.2) (layer F.Cu) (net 5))
 (segment (start 111.08 105.5) (end 111.33 105.75) (width 0.2) (layer F.Cu) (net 5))
 (segment (start 111.33 105.75) (end 111.33 107) (width 0.2) (layer F.Cu) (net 5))
 (segment (start 111.25 108.5) (end 111.25 108.3) (width 0.2) (layer F.Cu) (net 6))
 (segment (start 111.25 108.3) (end 112.55 107) (width 0.2) (layer F.Cu) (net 6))
 (segment (start 112.55 107) (end 112.83 107) (width 0.2) (layer F.Cu) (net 6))
 (segment (start 113.08 104.25) (end 113.08 105.5) (width 0.2) (layer F.Cu) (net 6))
 (segment (start 113.08 105.5) (end 112.83 105.75) (width 0.2) (layer F.Cu) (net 6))
 (segment (start 112.83 105.75) (end 112.83 107) (width 0.2) (layer F.Cu) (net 6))
 (segment (start 108.28 103.88) (end 108.28 105.45) (width 0.25) (layer F.Cu) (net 1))
 (segment (start 108.56 105.54) (end 108.2 105.54) (width 0.25) (layer F.Cu) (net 1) (status 30))
 (segment (start 116.28 102.2) (end 116.28 104.15) (width 0.2) (layer F.Cu) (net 8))
 (segment (start 116.28 104.15) (end 116.73 104.6) (width 0.2) (layer F.Cu) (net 8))
 (segment (start 116.28 102.4) (end 116.28 102.2) (width 0.25) (layer F.Cu) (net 8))
 (segment (start 116.28 102.7) (end 116.28 102.2) (width 0.25) (layer F.Cu) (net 8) (status 30))
 (segment (start 116.73 104.6) (end 116.68 104.55) (width 0.25) (layer F.Cu) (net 8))
 (segment (start 110.08 103.75) (end 109.879999 103.549999) (width 0.2) (layer B.Cu) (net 9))
 (segment (start 114.33 103.75) (end 110.08 103.75) (width 0.2) (layer B.Cu) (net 9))
 (segment (start 111.08 103.25) (end 109.58 103.25) (width 0.2) (layer F.Cu) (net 9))
 (via (at 109.58 103.25) (size 0.6) (drill 0.4) (layers F.Cu B.Cu) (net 9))
 (segment (start 109.879999 103.549999) (end 109.58 103.25) (width 0.2) (layer B.Cu) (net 9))
 (segment (start 114.33 103.75) (end 115.18 104.6) (width 0.2) (layer F.Cu) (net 9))
 (via (at 114.33 103.75) (size 0.6) (drill 0.4) (layers F.Cu B.Cu) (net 9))
 (segment (start 115.18 104.6) (end 115.23 104.6) (width 0.2) (layer F.Cu) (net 9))
 (segment (start 115.23 104.6) (end 115.23 104.45) (width 0.25) (layer F.Cu) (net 9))
 (segment (start 115.23 104.6) (end 115.23 104.6) (width 0.25) (layer F.Cu) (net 9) (status 30))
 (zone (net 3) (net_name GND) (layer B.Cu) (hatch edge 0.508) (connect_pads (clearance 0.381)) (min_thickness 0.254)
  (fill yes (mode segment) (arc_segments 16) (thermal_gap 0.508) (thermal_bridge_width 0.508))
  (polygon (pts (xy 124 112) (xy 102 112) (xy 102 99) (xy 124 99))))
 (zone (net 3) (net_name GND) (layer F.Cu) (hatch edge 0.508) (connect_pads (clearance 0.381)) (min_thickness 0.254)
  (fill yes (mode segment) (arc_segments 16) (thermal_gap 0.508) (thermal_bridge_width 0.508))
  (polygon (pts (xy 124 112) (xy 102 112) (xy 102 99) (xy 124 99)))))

